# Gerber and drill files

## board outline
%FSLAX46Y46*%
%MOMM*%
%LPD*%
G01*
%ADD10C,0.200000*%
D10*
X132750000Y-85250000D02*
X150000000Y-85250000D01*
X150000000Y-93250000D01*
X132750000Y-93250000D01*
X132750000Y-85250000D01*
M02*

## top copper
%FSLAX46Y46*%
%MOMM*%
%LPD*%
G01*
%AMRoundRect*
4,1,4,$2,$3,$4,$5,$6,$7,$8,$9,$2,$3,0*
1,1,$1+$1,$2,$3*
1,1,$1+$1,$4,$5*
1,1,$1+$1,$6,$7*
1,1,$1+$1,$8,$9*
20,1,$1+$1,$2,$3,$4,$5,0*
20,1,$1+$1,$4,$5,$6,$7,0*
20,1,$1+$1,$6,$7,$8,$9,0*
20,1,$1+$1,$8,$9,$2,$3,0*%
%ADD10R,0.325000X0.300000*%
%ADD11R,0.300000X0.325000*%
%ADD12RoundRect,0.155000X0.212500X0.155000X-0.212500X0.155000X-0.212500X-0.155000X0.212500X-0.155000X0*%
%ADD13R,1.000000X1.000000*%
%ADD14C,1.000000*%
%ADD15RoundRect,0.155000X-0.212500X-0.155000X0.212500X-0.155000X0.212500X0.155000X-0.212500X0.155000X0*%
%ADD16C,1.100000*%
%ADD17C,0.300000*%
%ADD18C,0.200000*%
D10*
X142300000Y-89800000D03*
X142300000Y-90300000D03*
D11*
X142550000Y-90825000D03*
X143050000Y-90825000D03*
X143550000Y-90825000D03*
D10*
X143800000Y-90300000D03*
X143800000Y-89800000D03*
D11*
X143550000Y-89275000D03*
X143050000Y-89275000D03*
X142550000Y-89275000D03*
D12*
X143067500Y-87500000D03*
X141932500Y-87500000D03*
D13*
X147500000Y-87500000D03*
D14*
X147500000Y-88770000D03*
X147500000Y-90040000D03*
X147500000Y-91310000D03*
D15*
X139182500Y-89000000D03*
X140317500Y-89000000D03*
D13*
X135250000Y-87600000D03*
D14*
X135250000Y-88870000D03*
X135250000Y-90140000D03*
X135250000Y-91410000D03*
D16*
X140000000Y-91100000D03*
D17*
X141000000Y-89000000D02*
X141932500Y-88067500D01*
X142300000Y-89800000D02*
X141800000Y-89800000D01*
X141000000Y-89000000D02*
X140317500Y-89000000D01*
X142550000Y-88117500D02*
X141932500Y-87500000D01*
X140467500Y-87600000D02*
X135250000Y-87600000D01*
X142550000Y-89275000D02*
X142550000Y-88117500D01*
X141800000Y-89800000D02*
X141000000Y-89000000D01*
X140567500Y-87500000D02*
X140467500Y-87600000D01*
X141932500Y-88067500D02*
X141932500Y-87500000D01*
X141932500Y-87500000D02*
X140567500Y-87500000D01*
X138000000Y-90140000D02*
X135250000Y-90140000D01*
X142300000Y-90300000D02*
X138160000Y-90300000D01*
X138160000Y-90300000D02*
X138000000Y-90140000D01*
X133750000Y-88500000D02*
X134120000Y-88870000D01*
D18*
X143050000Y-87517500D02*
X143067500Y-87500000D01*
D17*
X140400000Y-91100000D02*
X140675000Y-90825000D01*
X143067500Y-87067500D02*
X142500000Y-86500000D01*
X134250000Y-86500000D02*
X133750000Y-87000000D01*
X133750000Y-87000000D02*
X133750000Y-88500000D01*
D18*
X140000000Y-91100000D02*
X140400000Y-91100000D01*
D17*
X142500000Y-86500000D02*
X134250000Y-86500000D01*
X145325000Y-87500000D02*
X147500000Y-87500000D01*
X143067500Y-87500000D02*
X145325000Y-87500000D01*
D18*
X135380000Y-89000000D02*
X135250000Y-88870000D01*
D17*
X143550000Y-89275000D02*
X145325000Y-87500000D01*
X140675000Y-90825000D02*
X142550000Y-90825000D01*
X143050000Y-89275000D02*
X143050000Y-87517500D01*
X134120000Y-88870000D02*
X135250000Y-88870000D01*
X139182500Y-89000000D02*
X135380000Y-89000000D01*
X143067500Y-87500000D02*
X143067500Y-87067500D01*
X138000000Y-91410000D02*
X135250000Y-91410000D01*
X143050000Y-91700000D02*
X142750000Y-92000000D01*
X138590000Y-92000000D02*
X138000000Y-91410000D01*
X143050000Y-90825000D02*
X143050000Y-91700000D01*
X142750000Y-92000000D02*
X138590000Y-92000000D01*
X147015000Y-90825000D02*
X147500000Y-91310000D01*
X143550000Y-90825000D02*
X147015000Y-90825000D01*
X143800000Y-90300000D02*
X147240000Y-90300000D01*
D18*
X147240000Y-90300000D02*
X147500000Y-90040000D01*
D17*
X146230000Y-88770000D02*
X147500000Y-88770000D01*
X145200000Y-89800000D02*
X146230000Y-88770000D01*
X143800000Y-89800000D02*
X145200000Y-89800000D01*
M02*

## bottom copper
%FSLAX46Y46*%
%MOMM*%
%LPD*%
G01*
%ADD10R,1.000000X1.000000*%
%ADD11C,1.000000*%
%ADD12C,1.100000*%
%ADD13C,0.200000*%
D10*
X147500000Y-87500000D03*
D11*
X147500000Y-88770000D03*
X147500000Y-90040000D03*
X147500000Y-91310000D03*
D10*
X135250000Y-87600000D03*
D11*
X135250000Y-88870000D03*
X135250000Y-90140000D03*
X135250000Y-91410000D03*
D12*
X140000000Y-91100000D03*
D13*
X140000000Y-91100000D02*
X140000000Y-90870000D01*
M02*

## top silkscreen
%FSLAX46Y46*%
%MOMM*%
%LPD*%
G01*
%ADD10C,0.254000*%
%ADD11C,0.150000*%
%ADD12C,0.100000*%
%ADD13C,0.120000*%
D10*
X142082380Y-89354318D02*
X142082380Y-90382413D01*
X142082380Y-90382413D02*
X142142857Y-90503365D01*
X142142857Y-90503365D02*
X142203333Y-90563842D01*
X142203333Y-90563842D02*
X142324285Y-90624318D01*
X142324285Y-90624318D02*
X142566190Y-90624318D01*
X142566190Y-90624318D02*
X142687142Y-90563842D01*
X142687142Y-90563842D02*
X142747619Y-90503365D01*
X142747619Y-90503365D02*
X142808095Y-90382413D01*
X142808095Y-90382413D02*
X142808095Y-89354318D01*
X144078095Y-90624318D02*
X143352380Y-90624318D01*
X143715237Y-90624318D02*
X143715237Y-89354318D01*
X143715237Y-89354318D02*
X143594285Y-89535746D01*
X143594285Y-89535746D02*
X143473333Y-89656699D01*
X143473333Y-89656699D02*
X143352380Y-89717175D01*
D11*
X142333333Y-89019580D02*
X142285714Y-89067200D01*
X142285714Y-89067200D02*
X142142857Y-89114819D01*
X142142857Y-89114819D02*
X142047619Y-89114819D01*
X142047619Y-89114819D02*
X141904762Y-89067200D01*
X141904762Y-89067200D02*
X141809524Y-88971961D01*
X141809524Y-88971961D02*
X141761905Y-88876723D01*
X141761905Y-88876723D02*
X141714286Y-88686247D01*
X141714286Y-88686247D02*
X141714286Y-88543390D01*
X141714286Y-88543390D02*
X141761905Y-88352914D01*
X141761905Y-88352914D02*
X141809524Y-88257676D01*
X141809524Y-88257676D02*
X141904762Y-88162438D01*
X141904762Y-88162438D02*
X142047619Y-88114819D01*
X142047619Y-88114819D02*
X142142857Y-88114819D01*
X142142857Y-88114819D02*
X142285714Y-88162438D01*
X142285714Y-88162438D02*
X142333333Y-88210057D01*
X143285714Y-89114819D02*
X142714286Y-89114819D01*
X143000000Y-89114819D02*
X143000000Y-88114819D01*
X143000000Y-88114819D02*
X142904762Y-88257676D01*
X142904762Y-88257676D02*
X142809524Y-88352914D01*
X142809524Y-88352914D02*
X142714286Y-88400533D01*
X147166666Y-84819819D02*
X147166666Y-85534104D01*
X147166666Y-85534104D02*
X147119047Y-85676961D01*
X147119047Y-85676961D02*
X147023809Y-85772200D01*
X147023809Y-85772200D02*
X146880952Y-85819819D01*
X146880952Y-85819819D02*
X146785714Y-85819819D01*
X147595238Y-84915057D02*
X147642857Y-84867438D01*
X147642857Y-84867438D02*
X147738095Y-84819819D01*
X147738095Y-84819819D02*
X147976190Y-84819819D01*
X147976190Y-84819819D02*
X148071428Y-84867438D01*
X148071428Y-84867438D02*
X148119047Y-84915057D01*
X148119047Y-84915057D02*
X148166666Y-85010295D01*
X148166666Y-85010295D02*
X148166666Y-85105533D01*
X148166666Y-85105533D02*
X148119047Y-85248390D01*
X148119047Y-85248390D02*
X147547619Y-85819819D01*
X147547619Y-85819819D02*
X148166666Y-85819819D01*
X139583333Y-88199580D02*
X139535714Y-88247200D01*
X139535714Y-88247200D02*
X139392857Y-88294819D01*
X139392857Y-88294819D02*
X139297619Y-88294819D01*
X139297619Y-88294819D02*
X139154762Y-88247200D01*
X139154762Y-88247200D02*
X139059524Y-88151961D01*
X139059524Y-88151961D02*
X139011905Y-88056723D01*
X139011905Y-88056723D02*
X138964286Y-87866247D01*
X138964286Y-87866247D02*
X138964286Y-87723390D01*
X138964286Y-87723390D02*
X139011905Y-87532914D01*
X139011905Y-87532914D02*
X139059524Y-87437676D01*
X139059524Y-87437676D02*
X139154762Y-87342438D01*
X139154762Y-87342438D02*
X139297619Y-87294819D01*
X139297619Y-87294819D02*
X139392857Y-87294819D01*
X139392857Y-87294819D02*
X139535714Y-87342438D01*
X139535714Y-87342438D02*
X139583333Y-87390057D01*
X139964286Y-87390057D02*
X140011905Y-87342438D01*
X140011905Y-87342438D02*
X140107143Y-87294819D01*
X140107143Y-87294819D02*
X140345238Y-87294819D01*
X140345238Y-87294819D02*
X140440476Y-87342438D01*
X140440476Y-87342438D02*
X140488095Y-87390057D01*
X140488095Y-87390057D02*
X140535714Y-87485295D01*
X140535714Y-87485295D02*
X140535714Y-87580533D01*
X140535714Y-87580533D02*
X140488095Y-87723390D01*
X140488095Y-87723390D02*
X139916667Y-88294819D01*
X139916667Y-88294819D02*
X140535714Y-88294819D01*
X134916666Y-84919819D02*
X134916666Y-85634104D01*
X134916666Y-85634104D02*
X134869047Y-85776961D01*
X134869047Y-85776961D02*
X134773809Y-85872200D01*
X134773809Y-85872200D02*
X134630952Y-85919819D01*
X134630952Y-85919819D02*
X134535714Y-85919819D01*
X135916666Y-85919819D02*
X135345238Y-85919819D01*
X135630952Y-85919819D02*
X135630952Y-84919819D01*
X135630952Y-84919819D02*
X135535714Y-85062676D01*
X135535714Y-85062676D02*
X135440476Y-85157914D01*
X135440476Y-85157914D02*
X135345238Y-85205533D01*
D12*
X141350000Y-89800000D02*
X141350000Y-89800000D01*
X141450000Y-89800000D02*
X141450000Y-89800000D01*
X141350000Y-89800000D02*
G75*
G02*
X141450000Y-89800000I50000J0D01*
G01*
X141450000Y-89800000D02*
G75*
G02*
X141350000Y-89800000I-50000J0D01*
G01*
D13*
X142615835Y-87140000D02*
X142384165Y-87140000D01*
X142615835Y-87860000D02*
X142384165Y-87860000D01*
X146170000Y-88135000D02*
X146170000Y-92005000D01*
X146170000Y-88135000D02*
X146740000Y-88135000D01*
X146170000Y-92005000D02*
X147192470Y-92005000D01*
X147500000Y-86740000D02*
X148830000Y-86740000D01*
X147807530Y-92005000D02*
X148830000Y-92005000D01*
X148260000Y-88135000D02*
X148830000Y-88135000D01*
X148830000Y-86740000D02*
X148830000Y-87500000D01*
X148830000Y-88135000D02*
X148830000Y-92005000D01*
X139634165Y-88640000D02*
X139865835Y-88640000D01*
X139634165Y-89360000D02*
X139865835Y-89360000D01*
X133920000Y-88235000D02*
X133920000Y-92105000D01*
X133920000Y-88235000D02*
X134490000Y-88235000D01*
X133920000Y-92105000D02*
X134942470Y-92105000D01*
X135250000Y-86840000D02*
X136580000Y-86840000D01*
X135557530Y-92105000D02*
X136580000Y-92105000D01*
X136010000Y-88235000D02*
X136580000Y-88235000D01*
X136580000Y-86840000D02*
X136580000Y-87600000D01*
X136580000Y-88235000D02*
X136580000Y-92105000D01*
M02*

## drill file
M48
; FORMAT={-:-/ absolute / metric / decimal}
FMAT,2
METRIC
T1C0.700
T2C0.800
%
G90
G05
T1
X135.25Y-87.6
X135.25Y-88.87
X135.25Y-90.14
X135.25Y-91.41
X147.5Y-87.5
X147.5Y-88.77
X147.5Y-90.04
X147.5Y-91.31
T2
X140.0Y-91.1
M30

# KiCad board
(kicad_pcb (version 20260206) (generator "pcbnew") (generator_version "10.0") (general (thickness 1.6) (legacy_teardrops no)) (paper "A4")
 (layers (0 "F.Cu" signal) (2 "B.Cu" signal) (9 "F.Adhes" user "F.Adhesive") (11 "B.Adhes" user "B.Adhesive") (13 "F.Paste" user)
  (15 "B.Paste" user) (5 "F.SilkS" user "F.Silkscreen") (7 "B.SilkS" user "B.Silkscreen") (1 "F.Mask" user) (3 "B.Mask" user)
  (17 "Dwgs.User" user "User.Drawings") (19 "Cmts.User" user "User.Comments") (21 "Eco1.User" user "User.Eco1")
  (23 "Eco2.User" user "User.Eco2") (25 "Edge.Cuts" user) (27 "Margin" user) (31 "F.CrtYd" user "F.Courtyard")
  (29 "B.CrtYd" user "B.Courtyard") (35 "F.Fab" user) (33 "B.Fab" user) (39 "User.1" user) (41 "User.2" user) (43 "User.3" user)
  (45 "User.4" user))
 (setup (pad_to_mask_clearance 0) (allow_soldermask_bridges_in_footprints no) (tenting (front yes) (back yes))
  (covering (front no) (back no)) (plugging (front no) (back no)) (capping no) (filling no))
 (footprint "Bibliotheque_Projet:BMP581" (layer "F.Cu") (at 143.05 90.05)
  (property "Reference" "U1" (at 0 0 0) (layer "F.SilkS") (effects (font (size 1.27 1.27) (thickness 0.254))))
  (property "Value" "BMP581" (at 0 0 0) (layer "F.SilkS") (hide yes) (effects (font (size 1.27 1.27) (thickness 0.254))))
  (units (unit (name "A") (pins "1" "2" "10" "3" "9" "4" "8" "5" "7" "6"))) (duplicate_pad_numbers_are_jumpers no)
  (fp_line (start -1.7 -0.25) (end -1.7 -0.25) (stroke (width 0.1) (type solid)) (layer "F.SilkS"))
  (fp_line (start -1.6 -0.25) (end -1.6 -0.25) (stroke (width 0.1) (type solid)) (layer "F.SilkS"))
  (fp_arc (start -1.7 -0.25) (mid -1.65 -0.3) (end -1.6 -0.25) (stroke (width 0.1) (type solid)) (layer "F.SilkS"))
  (fp_arc (start -1.6 -0.25) (mid -1.65 -0.2) (end -1.7 -0.25) (stroke (width 0.1) (type solid)) (layer "F.SilkS"))
  (pad "1" smd rect (at -0.75 -0.25 90) (size 0.3 0.325) (layers "F.Cu" "F.Mask" "F.Paste") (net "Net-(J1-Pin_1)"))
  (pad "2" smd rect (at -0.75 0.25 90) (size 0.3 0.325) (layers "F.Cu" "F.Mask" "F.Paste") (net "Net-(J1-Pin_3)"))
  (pad "3" smd rect (at -0.5 0.775) (size 0.3 0.325) (layers "F.Cu" "F.Mask" "F.Paste") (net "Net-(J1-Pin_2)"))
  (pad "4" smd rect (at 0 0.775) (size 0.3 0.325) (layers "F.Cu" "F.Mask" "F.Paste") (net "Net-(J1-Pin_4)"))
  (pad "5" smd rect (at 0.5 0.775) (size 0.3 0.325) (layers "F.Cu" "F.Mask" "F.Paste") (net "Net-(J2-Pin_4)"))
  (pad "6" smd rect (at 0.75 0.25 90) (size 0.3 0.325) (layers "F.Cu" "F.Mask" "F.Paste") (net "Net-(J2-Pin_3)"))
  (pad "7" smd rect (at 0.75 -0.25 90) (size 0.3 0.325) (layers "F.Cu" "F.Mask" "F.Paste") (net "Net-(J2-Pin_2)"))
  (pad "8" smd rect (at 0.5 -0.775) (size 0.3 0.325) (layers "F.Cu" "F.Mask" "F.Paste") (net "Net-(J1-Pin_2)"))
  (pad "9" smd rect (at 0 -0.775) (size 0.3 0.325) (layers "F.Cu" "F.Mask" "F.Paste") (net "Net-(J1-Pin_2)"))
  (pad "10" smd rect (at -0.5 -0.775) (size 0.3 0.325) (layers "F.Cu" "F.Mask" "F.Paste") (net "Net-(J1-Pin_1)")))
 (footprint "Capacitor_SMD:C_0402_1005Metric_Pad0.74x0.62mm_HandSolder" (layer "F.Cu") (at 142.5 87.5 180)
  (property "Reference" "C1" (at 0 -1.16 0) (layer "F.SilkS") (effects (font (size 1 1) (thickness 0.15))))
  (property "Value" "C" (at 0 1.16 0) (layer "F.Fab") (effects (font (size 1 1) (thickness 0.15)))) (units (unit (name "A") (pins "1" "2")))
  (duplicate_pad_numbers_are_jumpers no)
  (fp_line (start -0.115835 0.36) (end 0.115835 0.36) (stroke (width 0.12) (type solid)) (layer "F.SilkS"))
  (fp_line (start -0.115835 -0.36) (end 0.115835 -0.36) (stroke (width 0.12) (type solid)) (layer "F.SilkS"))
  (pad "1" smd roundrect (at -0.5675 0 180) (size 0.735 0.62) (layers "F.Cu" "F.Mask" "F.Paste") (roundrect_rratio 0.25)
   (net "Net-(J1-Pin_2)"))
  (pad "2" smd roundrect (at 0.5675 0 180) (size 0.735 0.62) (layers "F.Cu" "F.Mask" "F.Paste") (roundrect_rratio 0.25)
   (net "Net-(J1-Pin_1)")))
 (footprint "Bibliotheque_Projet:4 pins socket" (layer "F.Cu") (at 147.5 87.5)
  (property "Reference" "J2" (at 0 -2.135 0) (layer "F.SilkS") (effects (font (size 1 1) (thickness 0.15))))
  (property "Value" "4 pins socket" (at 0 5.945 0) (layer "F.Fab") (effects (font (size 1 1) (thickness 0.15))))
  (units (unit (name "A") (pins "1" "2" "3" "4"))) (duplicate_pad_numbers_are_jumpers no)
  (fp_line (start -1.33 0.635) (end -1.33 4.505) (stroke (width 0.12) (type solid)) (layer "F.SilkS"))
  (fp_line (start -1.33 0.635) (end -0.76 0.635) (stroke (width 0.12) (type solid)) (layer "F.SilkS"))
  (fp_line (start -1.33 4.505) (end -0.30753 4.505) (stroke (width 0.12) (type solid)) (layer "F.SilkS"))
  (fp_line (start 0 -0.76) (end 1.33 -0.76) (stroke (width 0.12) (type solid)) (layer "F.SilkS"))
  (fp_line (start 0.30753 4.505) (end 1.33 4.505) (stroke (width 0.12) (type solid)) (layer "F.SilkS"))
  (fp_line (start 0.76 0.635) (end 1.33 0.635) (stroke (width 0.12) (type solid)) (layer "F.SilkS"))
  (fp_line (start 1.33 -0.76) (end 1.33 0) (stroke (width 0.12) (type solid)) (layer "F.SilkS"))
  (fp_line (start 1.33 0.635) (end 1.33 4.505) (stroke (width 0.12) (type solid)) (layer "F.SilkS"))
  (pad "1" thru_hole rect (at 0 0) (size 1 1) (drill 0.7) (layers "*.Cu" "*.Mask") (remove_unused_layers no) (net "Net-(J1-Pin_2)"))
  (pad "2" thru_hole circle (at 0 1.27) (size 1 1) (drill 0.7) (layers "*.Cu" "*.Mask") (remove_unused_layers no) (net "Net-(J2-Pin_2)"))
  (pad "3" thru_hole circle (at 0 2.54) (size 1 1) (drill 0.7) (layers "*.Cu" "*.Mask") (remove_unused_layers no) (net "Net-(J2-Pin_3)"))
  (pad "4" thru_hole circle (at 0 3.81) (size 1 1) (drill 0.7) (layers "*.Cu" "*.Mask") (remove_unused_layers no) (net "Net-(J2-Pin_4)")))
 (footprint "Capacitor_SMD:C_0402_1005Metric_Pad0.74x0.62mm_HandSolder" (layer "F.Cu") (at 139.75 89)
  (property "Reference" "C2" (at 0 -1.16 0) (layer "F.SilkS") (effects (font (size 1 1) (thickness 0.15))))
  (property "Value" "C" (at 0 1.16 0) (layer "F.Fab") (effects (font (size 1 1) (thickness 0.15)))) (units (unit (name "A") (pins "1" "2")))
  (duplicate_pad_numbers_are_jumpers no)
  (fp_line (start -0.115835 -0.36) (end 0.115835 -0.36) (stroke (width 0.12) (type solid)) (layer "F.SilkS"))
  (fp_line (start -0.115835 0.36) (end 0.115835 0.36) (stroke (width 0.12) (type solid)) (layer "F.SilkS"))
  (pad "1" smd roundrect (at -0.5675 0) (size 0.735 0.62) (layers "F.Cu" "F.Mask" "F.Paste") (roundrect_rratio 0.25) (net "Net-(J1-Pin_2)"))
  (pad "2" smd roundrect (at 0.5675 0) (size 0.735 0.62) (layers "F.Cu" "F.Mask" "F.Paste") (roundrect_rratio 0.25) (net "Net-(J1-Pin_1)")))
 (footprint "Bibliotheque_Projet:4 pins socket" (layer "F.Cu") (at 135.25 87.6)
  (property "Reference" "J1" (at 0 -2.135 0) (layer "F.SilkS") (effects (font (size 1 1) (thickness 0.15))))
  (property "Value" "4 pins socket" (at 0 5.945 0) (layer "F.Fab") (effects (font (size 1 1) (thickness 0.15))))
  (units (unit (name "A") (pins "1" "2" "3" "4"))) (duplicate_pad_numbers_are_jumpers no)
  (fp_line (start -1.33 0.635) (end -1.33 4.505) (stroke (width 0.12) (type solid)) (layer "F.SilkS"))
  (fp_line (start -1.33 0.635) (end -0.76 0.635) (stroke (width 0.12) (type solid)) (layer "F.SilkS"))
  (fp_line (start -1.33 4.505) (end -0.30753 4.505) (stroke (width 0.12) (type solid)) (layer "F.SilkS"))
  (fp_line (start 0 -0.76) (end 1.33 -0.76) (stroke (width 0.12) (type solid)) (layer "F.SilkS"))
  (fp_line (start 0.30753 4.505) (end 1.33 4.505) (stroke (width 0.12) (type solid)) (layer "F.SilkS"))
  (fp_line (start 0.76 0.635) (end 1.33 0.635) (stroke (width 0.12) (type solid)) (layer "F.SilkS"))
  (fp_line (start 1.33 -0.76) (end 1.33 0) (stroke (width 0.12) (type solid)) (layer "F.SilkS"))
  (fp_line (start 1.33 0.635) (end 1.33 4.505) (stroke (width 0.12) (type solid)) (layer "F.SilkS"))
  (pad "1" thru_hole rect (at 0 0) (size 1 1) (drill 0.7) (layers "*.Cu" "*.Mask") (remove_unused_layers no) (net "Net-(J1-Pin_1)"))
  (pad "2" thru_hole circle (at 0 1.27) (size 1 1) (drill 0.7) (layers "*.Cu" "*.Mask") (remove_unused_layers no) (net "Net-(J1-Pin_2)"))
  (pad "3" thru_hole circle (at 0 2.54) (size 1 1) (drill 0.7) (layers "*.Cu" "*.Mask") (remove_unused_layers no) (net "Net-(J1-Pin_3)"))
  (pad "4" thru_hole circle (at 0 3.81) (size 1 1) (drill 0.7) (layers "*.Cu" "*.Mask") (remove_unused_layers no) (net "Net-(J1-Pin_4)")))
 (gr_rect (start 132.75 85.25) (end 150 93.25) (stroke (width 0.2) (type solid)) (fill no) (layer "Edge.Cuts"))
 (segment (start 141 89) (end 141.9325 88.0675) (width 0.3) (layer "F.Cu") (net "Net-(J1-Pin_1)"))
 (segment (start 142.3 89.8) (end 141.8 89.8) (width 0.3) (layer "F.Cu") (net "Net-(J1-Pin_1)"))
 (segment (start 141 89) (end 140.3175 89) (width 0.3) (layer "F.Cu") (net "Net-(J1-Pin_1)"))
 (segment (start 142.55 88.1175) (end 141.9325 87.5) (width 0.3) (layer "F.Cu") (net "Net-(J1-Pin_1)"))
 (segment (start 140.4675 87.6) (end 135.25 87.6) (width 0.3) (layer "F.Cu") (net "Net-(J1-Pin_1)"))
 (segment (start 142.55 89.275) (end 142.55 88.1175) (width 0.3) (layer "F.Cu") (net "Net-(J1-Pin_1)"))
 (segment (start 141.8 89.8) (end 141 89) (width 0.3) (layer "F.Cu") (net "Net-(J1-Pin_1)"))
 (segment (start 140.5675 87.5) (end 140.4675 87.6) (width 0.3) (layer "F.Cu") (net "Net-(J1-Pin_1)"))
 (segment (start 141.9325 88.0675) (end 141.9325 87.5) (width 0.3) (layer "F.Cu") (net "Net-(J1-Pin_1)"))
 (segment (start 141.9325 87.5) (end 140.5675 87.5) (width 0.3) (layer "F.Cu") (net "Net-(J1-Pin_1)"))
 (segment (start 138 90.14) (end 135.25 90.14) (width 0.3) (layer "F.Cu") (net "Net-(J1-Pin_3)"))
 (segment (start 142.3 90.3) (end 138.16 90.3) (width 0.3) (layer "F.Cu") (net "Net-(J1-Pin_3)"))
 (segment (start 138.16 90.3) (end 138 90.14) (width 0.3) (layer "F.Cu") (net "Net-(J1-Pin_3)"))
 (segment (start 133.75 88.5) (end 134.12 88.87) (width 0.3) (layer "F.Cu") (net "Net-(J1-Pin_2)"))
 (segment (start 143.05 87.5175) (end 143.0675 87.5) (width 0.2) (layer "F.Cu") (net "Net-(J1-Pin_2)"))
 (segment (start 140.4 91.1) (end 140.675 90.825) (width 0.3) (layer "F.Cu") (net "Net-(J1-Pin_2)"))
 (segment (start 143.0675 87.0675) (end 142.5 86.5) (width 0.3) (layer "F.Cu") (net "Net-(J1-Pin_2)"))
 (segment (start 134.25 86.5) (end 133.75 87) (width 0.3) (layer "F.Cu") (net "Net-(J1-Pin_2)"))
 (segment (start 133.75 87) (end 133.75 88.5) (width 0.3) (layer "F.Cu") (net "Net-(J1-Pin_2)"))
 (segment (start 140 91.1) (end 140.4 91.1) (width 0.2) (layer "F.Cu") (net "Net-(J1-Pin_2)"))
 (segment (start 142.5 86.5) (end 134.25 86.5) (width 0.3) (layer "F.Cu") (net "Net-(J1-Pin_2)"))
 (segment (start 145.325 87.5) (end 147.5 87.5) (width 0.3) (layer "F.Cu") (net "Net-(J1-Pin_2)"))
 (segment (start 143.0675 87.5) (end 145.325 87.5) (width 0.3) (layer "F.Cu") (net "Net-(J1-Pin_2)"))
 (segment (start 135.38 89) (end 135.25 88.87) (width 0.2) (layer "F.Cu") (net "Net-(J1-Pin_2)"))
 (segment (start 143.55 89.275) (end 145.325 87.5) (width 0.3) (layer "F.Cu") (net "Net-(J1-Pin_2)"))
 (segment (start 140.675 90.825) (end 142.55 90.825) (width 0.3) (layer "F.Cu") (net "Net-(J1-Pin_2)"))
 (segment (start 143.05 89.275) (end 143.05 87.5175) (width 0.3) (layer "F.Cu") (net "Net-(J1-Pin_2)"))
 (segment (start 134.12 88.87) (end 135.25 88.87) (width 0.3) (layer "F.Cu") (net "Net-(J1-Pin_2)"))
 (segment (start 139.1825 89) (end 135.38 89) (width 0.3) (layer "F.Cu") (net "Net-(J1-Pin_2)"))
 (segment (start 143.0675 87.5) (end 143.0675 87.0675) (width 0.3) (layer "F.Cu") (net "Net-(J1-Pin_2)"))
 (via (at 140 91.1) (size 1.1) (drill 0.8) (layers "F.Cu" "B.Cu") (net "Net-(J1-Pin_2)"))
 (segment (start 140 91.1) (end 140 90.87) (width 0.2) (layer "B.Cu") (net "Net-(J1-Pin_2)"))
 (segment (start 138 91.41) (end 135.25 91.41) (width 0.3) (layer "F.Cu") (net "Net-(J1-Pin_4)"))
 (segment (start 143.05 91.7) (end 142.75 92) (width 0.3) (layer "F.Cu") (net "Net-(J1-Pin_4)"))
 (segment (start 138.59 92) (end 138 91.41) (width 0.3) (layer "F.Cu") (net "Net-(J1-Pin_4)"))
 (segment (start 143.05 90.825) (end 143.05 91.7) (width 0.3) (layer "F.Cu") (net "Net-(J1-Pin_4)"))
 (segment (start 142.75 92) (end 138.59 92) (width 0.3) (layer "F.Cu") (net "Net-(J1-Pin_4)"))
 (segment (start 147.015 90.825) (end 147.5 91.31) (width 0.3) (layer "F.Cu") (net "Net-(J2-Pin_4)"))
 (segment (start 143.55 90.825) (end 147.015 90.825) (width 0.3) (layer "F.Cu") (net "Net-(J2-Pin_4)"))
 (segment (start 143.8 90.3) (end 147.24 90.3) (width 0.3) (layer "F.Cu") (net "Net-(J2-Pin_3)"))
 (segment (start 147.24 90.3) (end 147.5 90.04) (width 0.2) (layer "F.Cu") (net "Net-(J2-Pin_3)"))
 (segment (start 146.23 88.77) (end 147.5 88.77) (width 0.3) (layer "F.Cu") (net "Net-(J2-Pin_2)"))
 (segment (start 145.2 89.8) (end 146.23 88.77) (width 0.3) (layer "F.Cu") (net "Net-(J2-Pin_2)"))
 (segment (start 143.8 89.8) (end 145.2 89.8) (width 0.3) (layer "F.Cu") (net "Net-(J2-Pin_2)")))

